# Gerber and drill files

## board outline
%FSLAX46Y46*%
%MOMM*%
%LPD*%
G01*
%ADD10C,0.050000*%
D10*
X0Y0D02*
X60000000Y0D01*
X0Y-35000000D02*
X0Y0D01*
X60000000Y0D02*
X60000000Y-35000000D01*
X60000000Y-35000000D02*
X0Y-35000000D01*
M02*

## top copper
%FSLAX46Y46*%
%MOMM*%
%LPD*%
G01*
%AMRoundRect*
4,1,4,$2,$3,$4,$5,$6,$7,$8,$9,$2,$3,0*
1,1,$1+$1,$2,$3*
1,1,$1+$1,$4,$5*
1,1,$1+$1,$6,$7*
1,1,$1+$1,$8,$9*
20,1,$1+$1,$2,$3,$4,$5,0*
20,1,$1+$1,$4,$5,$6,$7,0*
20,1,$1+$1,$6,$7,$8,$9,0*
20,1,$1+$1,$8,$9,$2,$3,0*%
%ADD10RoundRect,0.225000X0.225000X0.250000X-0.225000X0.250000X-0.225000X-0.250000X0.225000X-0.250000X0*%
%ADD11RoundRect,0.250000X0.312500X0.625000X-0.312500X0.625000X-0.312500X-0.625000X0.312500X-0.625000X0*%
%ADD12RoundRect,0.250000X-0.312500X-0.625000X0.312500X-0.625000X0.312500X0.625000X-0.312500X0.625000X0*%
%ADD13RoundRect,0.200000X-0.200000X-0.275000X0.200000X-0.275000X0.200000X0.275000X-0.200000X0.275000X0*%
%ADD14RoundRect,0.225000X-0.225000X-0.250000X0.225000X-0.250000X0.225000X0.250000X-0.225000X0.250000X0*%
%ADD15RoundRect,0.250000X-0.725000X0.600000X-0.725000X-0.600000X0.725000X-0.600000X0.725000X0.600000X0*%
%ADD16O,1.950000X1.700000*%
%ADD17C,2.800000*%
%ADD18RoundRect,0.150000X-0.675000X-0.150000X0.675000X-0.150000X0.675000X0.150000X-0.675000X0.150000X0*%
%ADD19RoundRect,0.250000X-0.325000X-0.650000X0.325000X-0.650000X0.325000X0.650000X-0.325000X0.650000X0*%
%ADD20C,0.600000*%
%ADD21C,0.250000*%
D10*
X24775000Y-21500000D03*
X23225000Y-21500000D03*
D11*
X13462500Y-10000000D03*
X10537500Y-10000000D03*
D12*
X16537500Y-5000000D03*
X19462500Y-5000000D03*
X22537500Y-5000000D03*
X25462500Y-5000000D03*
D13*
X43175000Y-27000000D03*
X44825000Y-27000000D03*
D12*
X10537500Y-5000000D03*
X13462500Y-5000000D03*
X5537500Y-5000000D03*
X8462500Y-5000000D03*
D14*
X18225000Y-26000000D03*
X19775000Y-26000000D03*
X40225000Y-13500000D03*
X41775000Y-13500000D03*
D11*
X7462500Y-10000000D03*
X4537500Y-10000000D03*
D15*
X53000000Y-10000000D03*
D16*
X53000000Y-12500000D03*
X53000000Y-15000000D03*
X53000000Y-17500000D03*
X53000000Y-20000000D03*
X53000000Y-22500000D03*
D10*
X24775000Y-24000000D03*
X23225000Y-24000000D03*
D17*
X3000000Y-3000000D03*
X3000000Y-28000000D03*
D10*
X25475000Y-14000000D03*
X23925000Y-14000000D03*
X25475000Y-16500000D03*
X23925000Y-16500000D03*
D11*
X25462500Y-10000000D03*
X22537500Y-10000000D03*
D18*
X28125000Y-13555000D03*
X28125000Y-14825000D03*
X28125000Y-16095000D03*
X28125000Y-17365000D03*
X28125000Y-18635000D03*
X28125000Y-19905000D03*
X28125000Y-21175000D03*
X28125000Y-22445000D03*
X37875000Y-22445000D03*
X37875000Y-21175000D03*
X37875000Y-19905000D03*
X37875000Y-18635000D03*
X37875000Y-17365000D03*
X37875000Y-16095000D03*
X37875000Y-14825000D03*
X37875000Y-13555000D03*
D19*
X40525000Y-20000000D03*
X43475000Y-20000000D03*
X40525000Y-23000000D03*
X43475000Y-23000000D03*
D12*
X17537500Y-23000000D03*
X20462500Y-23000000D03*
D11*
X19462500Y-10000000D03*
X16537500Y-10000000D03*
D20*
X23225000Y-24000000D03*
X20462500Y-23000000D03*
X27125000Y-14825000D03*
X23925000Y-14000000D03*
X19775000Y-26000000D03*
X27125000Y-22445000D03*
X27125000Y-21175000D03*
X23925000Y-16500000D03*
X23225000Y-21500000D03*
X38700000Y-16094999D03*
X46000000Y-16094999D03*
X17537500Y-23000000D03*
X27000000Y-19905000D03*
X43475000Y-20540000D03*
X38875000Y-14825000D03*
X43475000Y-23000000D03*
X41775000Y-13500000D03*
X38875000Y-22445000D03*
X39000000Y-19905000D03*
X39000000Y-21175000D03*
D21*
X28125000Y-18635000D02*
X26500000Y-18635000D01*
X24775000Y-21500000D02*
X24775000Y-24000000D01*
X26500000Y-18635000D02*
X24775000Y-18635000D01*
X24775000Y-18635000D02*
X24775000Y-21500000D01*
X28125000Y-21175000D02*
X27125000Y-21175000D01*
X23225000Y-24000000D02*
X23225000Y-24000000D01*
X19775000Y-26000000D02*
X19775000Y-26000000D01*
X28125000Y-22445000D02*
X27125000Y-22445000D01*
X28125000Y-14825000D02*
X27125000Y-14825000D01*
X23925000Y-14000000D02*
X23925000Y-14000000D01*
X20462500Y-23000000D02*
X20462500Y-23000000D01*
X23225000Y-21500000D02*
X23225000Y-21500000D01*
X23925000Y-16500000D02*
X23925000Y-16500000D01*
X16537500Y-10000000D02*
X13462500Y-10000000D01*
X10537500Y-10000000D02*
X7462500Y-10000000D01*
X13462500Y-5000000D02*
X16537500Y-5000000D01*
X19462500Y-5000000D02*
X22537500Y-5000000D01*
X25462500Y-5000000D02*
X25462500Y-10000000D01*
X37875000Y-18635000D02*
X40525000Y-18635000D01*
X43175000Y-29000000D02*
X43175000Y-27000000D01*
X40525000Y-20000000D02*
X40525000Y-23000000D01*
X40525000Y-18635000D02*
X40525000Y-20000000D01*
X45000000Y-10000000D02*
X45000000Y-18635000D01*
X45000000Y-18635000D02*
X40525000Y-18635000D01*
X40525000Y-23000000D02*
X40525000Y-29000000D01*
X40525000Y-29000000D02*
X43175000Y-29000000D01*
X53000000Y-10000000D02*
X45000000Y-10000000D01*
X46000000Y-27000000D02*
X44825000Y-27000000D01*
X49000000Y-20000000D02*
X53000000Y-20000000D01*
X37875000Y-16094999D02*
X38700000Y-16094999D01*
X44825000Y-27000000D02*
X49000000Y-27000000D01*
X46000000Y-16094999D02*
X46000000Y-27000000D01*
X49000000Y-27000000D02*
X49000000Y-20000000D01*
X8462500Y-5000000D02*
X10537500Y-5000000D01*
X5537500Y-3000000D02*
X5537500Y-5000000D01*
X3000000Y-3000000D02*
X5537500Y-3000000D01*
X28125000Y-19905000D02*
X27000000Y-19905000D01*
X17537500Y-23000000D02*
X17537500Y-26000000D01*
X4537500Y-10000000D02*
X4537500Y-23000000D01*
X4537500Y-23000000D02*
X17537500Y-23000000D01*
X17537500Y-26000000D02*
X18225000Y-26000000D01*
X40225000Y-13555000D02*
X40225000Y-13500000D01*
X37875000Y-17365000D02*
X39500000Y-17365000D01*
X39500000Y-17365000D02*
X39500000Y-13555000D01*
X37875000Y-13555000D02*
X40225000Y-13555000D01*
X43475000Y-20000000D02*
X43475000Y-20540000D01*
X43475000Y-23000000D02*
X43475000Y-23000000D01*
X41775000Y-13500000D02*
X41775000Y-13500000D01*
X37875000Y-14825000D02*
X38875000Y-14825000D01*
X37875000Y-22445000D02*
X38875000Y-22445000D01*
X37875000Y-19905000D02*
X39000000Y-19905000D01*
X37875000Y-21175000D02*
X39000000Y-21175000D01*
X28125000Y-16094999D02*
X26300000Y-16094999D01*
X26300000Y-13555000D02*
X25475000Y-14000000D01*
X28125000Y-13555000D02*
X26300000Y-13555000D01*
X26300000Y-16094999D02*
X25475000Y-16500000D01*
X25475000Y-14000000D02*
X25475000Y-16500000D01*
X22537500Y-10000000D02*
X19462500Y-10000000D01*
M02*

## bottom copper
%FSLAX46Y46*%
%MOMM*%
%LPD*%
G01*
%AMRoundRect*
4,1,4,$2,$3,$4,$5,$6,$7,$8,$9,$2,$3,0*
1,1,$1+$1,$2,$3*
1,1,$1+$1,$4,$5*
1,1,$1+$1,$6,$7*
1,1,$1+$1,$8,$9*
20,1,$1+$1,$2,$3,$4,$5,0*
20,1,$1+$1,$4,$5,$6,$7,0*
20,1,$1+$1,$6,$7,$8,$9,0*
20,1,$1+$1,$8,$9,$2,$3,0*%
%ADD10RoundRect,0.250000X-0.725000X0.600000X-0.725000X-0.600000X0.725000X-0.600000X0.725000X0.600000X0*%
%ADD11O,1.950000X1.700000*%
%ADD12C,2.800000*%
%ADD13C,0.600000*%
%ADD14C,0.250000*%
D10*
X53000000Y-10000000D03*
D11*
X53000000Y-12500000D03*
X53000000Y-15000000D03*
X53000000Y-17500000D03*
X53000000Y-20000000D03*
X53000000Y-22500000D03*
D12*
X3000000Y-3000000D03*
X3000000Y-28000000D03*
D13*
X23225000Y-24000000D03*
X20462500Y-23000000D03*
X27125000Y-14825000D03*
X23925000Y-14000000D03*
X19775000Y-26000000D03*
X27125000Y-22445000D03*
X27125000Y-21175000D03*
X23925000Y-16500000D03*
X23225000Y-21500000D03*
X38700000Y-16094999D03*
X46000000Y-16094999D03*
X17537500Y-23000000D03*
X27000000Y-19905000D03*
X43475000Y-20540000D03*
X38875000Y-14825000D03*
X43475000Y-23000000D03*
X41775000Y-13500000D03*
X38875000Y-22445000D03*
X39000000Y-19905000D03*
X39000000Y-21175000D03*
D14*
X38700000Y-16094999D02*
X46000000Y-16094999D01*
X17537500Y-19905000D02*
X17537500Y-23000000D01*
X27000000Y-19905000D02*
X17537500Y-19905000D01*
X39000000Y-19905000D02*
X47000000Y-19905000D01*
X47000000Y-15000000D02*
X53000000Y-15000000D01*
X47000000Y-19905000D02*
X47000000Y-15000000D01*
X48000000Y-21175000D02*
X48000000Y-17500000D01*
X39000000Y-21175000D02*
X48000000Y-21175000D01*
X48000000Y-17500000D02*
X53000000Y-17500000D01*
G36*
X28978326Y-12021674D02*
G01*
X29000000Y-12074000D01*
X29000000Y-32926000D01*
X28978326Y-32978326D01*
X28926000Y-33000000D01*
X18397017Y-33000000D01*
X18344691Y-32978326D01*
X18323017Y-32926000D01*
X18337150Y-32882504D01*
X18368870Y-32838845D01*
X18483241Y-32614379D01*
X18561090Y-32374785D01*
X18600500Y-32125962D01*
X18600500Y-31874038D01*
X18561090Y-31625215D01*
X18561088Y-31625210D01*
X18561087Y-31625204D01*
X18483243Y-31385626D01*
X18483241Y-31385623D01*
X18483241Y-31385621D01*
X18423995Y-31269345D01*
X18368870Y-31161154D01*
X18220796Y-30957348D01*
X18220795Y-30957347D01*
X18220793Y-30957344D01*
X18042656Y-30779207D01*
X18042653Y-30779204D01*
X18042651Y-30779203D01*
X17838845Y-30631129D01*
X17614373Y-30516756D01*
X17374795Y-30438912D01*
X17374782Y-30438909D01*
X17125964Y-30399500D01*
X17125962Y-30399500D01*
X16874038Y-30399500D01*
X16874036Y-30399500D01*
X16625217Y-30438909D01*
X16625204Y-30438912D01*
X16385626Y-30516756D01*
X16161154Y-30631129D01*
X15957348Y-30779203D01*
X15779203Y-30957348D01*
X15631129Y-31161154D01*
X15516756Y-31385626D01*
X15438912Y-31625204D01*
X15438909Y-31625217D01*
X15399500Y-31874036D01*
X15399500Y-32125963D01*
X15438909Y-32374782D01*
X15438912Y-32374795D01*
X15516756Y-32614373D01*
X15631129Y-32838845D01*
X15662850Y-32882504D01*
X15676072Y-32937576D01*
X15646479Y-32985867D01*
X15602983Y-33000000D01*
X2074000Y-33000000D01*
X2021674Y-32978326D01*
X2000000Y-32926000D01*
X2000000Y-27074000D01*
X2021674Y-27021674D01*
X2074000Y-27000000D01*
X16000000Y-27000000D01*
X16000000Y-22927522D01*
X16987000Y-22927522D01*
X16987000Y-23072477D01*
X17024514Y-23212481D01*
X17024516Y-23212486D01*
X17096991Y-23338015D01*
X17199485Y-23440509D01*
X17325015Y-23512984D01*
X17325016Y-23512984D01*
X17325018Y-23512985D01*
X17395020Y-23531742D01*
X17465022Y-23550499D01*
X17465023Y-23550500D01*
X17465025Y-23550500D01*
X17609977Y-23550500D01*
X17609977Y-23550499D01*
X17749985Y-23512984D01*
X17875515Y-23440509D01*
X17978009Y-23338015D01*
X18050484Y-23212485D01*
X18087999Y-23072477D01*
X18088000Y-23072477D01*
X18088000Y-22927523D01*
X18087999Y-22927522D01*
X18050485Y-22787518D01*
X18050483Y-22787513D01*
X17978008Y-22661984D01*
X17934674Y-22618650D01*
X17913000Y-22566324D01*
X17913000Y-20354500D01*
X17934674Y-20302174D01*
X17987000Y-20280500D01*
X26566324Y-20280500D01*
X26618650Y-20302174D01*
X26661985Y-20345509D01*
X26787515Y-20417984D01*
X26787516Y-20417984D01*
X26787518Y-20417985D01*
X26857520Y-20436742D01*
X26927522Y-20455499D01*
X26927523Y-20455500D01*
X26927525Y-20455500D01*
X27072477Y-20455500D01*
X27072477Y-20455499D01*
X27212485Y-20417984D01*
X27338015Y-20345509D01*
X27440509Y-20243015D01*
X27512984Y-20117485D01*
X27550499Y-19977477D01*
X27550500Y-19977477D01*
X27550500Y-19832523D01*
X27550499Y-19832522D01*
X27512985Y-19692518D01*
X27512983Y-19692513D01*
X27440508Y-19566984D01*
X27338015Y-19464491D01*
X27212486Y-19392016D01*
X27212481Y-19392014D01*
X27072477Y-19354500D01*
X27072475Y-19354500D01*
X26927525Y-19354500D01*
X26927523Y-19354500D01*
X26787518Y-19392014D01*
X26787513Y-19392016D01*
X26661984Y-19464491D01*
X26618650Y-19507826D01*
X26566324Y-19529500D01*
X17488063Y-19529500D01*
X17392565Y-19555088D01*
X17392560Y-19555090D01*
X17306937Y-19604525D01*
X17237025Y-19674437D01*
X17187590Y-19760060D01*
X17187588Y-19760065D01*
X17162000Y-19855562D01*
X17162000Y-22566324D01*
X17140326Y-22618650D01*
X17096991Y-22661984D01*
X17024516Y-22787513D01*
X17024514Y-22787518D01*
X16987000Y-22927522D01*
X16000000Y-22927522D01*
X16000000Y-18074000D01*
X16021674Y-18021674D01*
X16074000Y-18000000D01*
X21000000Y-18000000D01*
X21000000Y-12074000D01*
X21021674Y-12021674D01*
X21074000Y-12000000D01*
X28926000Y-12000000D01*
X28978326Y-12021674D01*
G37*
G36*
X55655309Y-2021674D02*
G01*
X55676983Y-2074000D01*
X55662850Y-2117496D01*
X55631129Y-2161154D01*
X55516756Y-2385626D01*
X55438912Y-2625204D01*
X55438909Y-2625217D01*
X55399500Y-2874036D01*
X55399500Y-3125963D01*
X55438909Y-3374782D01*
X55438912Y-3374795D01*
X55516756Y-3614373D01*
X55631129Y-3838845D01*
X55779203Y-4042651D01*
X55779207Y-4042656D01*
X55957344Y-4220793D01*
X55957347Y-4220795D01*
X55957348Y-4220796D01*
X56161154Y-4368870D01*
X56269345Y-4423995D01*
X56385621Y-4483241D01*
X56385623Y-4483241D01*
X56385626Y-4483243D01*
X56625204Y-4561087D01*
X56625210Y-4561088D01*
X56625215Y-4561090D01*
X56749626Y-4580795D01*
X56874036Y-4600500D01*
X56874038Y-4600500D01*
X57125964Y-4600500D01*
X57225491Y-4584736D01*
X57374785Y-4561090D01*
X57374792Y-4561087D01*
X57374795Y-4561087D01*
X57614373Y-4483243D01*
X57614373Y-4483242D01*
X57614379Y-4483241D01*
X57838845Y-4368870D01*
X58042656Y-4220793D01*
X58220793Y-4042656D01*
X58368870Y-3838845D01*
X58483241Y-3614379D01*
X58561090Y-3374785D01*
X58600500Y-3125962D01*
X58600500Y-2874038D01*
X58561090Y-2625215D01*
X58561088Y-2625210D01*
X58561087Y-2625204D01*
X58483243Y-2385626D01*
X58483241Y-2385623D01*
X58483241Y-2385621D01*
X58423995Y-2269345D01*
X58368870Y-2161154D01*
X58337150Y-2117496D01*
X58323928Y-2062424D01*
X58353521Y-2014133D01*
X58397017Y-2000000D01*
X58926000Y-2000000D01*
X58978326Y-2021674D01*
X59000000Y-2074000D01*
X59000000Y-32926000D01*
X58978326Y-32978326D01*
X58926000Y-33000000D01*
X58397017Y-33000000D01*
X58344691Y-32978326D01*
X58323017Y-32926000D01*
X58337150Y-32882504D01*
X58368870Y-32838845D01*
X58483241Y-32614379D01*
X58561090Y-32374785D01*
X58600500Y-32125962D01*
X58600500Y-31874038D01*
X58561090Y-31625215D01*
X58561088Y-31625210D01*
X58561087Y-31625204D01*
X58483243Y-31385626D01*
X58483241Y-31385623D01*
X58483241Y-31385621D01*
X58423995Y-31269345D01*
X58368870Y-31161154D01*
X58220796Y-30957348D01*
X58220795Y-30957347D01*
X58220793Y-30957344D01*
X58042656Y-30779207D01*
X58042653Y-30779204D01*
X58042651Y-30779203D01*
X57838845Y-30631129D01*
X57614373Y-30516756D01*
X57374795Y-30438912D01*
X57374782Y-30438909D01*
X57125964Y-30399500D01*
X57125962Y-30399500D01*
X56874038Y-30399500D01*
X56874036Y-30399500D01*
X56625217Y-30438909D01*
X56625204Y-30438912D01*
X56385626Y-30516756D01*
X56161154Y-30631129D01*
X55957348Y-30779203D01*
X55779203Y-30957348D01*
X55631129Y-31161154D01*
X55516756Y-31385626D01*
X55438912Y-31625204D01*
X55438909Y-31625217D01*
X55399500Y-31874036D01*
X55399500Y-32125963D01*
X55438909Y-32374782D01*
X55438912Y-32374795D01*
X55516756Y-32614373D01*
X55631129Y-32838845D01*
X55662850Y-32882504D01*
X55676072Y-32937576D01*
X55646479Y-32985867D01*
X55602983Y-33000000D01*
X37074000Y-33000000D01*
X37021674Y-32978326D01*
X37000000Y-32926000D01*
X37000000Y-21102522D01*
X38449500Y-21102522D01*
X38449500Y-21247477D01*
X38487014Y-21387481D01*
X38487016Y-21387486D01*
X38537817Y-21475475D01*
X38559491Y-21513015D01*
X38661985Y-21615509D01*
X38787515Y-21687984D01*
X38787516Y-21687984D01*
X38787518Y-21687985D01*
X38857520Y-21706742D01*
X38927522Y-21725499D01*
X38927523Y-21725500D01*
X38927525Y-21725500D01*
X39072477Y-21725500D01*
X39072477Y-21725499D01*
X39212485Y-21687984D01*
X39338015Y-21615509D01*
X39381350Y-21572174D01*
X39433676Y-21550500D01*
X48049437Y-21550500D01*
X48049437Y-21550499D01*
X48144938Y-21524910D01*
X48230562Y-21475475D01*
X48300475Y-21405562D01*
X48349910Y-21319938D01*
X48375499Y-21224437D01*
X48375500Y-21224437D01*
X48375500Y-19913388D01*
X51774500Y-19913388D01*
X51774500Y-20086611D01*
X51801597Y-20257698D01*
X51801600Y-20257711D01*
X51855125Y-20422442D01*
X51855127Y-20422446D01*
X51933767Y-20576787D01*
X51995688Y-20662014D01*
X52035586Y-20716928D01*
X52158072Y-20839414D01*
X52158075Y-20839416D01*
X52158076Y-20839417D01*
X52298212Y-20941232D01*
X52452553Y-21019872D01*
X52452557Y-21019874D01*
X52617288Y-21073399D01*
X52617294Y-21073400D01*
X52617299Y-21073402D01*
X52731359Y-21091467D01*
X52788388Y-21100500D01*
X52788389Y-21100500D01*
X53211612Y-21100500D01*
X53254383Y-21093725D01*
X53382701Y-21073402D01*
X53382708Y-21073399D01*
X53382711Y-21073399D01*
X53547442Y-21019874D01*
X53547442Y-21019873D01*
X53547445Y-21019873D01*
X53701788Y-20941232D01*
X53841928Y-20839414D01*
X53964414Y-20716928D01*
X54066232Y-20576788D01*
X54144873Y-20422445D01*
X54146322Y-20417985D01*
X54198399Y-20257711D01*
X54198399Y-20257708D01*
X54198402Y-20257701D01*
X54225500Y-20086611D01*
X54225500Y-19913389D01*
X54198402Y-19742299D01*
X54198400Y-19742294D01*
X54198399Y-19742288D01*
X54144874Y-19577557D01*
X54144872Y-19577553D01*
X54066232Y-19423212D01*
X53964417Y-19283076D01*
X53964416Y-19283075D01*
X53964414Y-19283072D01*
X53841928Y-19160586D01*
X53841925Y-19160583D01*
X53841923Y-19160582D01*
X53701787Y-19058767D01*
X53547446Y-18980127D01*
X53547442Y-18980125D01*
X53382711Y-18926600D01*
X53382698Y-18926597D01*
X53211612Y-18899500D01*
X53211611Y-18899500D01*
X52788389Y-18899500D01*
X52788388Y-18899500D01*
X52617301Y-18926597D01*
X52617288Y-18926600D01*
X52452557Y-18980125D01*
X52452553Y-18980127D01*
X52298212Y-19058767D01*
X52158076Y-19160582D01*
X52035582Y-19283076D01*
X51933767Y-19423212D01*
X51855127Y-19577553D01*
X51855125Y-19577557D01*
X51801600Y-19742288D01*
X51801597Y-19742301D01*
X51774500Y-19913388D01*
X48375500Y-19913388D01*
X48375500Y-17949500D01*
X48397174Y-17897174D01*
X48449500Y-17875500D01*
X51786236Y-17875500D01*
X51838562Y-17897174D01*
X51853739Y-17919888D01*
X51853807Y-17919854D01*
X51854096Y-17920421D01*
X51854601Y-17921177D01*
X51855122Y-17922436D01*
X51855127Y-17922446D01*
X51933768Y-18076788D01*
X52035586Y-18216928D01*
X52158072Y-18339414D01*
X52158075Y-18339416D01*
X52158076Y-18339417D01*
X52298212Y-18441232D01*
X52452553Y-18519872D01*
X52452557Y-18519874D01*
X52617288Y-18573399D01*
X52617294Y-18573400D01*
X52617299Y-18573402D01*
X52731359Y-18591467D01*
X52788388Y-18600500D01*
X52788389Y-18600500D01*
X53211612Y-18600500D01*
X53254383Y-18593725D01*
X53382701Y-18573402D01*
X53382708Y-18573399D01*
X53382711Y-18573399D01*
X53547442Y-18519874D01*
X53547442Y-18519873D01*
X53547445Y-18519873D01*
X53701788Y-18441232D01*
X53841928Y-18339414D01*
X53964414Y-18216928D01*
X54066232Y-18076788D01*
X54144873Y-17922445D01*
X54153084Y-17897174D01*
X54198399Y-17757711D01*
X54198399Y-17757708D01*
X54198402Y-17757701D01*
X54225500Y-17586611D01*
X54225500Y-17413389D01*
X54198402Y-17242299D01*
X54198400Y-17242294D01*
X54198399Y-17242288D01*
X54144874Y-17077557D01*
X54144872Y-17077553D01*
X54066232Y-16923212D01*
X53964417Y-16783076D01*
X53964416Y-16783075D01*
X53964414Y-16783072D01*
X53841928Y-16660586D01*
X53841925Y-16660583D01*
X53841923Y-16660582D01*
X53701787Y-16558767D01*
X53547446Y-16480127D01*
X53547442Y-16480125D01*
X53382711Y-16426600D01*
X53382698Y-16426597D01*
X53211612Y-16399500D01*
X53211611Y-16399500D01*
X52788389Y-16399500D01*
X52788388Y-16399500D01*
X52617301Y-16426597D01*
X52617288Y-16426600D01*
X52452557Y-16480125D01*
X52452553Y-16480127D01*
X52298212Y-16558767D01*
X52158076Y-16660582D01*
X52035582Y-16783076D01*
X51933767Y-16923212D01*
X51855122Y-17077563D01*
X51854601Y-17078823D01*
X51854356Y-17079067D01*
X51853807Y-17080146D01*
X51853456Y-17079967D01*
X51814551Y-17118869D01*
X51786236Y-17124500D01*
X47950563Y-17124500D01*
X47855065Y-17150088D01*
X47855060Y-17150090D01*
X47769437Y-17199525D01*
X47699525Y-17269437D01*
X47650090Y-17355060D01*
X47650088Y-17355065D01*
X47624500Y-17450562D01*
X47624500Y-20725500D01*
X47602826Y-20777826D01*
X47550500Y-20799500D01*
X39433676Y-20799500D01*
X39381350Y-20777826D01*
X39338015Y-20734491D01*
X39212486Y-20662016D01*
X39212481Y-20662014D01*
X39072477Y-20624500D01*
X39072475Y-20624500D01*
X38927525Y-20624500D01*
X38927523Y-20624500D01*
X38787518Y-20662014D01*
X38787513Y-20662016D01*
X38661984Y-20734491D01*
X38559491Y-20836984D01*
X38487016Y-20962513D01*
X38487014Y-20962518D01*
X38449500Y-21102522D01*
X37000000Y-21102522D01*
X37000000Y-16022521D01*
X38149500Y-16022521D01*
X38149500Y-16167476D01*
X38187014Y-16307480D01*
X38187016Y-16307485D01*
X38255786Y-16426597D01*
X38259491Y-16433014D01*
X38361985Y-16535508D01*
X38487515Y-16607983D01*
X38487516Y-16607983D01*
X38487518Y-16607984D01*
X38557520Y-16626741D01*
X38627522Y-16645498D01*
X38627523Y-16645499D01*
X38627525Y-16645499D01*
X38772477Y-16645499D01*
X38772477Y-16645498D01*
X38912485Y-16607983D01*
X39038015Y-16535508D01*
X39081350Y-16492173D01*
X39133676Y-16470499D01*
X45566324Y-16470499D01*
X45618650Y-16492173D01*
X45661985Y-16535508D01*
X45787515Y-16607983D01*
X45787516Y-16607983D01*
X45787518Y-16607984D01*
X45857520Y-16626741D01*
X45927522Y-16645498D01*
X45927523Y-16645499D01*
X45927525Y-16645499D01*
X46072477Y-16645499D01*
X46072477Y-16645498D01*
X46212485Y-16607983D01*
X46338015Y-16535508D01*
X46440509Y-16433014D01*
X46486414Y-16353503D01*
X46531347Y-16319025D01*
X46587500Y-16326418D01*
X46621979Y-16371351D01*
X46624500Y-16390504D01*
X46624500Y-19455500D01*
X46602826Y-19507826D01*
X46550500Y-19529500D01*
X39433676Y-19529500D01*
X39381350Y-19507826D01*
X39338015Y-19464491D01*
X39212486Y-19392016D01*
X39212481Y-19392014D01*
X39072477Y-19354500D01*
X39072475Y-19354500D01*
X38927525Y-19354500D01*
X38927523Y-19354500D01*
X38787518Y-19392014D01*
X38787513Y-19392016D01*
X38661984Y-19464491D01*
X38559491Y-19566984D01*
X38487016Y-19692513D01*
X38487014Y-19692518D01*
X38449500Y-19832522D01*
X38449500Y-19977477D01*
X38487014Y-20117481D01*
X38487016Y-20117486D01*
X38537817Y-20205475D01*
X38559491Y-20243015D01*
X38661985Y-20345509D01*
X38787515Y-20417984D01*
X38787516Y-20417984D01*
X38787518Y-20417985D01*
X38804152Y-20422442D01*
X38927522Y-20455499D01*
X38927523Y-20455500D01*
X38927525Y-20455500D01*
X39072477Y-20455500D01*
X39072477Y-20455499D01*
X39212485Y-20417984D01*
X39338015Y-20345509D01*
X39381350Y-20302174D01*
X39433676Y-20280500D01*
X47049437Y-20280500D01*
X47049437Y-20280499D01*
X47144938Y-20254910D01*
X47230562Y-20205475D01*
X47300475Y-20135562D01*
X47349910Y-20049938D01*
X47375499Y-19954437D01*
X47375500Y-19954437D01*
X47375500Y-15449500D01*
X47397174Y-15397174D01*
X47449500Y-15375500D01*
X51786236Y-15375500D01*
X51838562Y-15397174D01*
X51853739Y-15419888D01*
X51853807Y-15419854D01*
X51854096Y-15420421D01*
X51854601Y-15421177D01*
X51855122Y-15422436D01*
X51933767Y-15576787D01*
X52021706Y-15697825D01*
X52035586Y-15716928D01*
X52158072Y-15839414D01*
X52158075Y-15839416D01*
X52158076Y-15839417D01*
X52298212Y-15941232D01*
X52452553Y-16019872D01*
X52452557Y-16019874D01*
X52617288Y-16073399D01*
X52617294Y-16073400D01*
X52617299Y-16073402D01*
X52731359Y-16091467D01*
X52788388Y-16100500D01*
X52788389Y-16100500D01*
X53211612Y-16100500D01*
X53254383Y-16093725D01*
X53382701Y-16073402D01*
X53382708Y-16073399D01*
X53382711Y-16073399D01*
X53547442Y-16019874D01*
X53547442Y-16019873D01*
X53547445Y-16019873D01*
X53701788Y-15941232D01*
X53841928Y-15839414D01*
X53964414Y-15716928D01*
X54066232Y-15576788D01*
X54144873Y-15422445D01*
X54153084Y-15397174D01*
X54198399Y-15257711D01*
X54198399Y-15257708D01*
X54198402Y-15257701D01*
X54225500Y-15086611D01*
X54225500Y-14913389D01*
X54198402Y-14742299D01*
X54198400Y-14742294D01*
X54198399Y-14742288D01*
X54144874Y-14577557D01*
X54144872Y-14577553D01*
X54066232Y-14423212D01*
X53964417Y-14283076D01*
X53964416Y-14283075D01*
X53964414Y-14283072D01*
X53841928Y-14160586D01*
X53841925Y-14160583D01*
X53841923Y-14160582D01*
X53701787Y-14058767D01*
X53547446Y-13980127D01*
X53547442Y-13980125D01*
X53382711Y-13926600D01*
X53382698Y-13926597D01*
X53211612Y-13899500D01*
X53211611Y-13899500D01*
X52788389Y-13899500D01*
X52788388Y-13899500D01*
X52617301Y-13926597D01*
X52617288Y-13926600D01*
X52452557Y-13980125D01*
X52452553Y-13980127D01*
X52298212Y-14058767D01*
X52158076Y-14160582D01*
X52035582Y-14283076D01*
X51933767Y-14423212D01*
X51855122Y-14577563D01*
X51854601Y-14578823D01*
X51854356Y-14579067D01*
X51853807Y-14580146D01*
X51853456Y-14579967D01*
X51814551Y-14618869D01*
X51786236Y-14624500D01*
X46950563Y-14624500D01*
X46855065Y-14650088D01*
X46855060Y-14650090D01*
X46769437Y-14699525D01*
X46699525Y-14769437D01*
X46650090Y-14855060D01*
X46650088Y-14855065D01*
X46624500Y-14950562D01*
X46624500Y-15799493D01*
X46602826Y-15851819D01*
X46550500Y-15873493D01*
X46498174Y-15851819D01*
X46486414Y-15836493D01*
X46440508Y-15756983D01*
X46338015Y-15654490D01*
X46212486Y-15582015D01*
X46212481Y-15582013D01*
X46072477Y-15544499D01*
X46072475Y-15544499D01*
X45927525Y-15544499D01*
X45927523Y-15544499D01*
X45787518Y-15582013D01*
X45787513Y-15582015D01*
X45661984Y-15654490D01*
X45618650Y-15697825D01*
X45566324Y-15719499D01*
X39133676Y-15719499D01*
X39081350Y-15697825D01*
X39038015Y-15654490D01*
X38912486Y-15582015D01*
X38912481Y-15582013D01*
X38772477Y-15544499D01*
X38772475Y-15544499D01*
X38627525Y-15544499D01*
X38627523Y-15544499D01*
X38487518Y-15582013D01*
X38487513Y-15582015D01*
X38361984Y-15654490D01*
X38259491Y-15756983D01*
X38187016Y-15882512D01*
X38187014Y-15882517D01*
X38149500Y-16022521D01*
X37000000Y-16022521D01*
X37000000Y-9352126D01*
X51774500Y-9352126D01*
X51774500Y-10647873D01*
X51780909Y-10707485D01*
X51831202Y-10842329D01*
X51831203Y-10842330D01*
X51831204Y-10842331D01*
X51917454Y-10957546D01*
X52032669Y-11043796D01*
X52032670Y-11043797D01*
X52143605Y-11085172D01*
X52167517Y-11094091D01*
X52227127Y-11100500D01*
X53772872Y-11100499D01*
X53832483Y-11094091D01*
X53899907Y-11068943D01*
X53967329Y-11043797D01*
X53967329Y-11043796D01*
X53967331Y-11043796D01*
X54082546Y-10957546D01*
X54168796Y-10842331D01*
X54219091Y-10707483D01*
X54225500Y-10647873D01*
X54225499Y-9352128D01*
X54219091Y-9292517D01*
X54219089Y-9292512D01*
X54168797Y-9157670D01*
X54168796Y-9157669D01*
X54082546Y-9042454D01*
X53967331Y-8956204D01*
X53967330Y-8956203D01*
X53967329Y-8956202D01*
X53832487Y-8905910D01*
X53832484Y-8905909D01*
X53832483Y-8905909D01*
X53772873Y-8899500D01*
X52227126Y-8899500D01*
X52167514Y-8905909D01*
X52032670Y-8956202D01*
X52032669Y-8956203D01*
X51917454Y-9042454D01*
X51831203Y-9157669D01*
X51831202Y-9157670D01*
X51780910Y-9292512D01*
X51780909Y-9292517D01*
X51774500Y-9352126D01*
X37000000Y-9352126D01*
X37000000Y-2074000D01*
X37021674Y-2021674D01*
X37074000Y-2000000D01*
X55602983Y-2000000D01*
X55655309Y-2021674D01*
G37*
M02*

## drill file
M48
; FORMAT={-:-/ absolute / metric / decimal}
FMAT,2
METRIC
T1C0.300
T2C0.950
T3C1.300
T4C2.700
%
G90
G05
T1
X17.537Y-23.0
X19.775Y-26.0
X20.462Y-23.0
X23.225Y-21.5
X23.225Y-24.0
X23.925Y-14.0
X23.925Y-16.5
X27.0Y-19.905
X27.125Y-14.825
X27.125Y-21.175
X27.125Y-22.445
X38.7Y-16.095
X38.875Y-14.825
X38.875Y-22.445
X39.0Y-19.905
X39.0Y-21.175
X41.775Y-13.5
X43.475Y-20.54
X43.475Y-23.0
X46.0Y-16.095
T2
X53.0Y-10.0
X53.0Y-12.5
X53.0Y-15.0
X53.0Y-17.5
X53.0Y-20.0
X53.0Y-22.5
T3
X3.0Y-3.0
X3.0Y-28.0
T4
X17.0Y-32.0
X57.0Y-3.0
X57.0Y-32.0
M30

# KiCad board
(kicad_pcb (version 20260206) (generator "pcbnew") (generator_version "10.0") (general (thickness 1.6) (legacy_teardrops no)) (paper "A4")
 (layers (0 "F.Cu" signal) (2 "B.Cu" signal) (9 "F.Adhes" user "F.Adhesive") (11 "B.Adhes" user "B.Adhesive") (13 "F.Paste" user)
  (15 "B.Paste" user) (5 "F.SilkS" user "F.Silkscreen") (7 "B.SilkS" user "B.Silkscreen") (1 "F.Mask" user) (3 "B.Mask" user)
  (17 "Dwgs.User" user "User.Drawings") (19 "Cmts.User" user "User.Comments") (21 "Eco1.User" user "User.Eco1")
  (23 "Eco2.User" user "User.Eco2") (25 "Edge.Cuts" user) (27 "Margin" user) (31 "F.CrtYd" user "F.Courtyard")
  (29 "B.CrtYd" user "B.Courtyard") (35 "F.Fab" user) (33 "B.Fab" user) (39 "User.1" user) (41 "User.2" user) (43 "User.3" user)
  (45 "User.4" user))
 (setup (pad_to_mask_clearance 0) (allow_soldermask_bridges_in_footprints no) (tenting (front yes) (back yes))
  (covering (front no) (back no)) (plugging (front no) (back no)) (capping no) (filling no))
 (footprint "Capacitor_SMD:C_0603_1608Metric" (layer "F.Cu") (at 24 21.5 180)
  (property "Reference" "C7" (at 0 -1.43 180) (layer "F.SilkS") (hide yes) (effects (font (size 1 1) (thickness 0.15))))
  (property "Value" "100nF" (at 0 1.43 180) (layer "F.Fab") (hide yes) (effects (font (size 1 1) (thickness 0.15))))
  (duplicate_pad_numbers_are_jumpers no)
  (pad "1" smd roundrect (at -0.775 0 180) (size 0.9 0.95) (layers "F.Cu" "F.Mask" "F.Paste") (roundrect_rratio 0.25) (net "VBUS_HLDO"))
  (pad "2" smd roundrect (at 0.775 0 180) (size 0.9 0.95) (layers "F.Cu" "F.Mask" "F.Paste") (roundrect_rratio 0.25) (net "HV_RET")))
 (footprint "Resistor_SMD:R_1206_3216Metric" (layer "F.Cu") (at 12 10 180)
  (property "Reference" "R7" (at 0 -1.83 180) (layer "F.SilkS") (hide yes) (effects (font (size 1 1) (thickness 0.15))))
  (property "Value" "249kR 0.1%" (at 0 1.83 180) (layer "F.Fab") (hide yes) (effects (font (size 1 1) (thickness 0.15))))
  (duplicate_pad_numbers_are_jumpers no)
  (pad "1" smd roundrect (at -1.4625 0 180) (size 1.125 1.75) (layers "F.Cu" "F.Mask" "F.Paste") (roundrect_rratio 0.222222)
   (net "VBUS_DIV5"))
  (pad "2" smd roundrect (at 1.4625 0 180) (size 1.125 1.75) (layers "F.Cu" "F.Mask" "F.Paste") (roundrect_rratio 0.222222)
   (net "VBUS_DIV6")))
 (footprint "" (layer "F.Cu") (at 57 32)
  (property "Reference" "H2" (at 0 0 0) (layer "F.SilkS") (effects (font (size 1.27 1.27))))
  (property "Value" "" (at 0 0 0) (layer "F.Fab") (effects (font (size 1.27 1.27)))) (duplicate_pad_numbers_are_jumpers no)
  (pad "" np_thru_hole circle (at 0 0) (size 2.7 2.7) (drill 2.7) (layers "*.Cu")))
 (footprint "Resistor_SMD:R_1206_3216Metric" (layer "F.Cu") (at 18 5)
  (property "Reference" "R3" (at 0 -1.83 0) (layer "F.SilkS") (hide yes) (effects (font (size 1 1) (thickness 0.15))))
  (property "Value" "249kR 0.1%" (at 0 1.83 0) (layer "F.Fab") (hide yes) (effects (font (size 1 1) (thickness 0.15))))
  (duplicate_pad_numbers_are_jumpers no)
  (pad "1" smd roundrect (at -1.4625 0) (size 1.125 1.75) (layers "F.Cu" "F.Mask" "F.Paste") (roundrect_rratio 0.222222) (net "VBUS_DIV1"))
  (pad "2" smd roundrect (at 1.4625 0) (size 1.125 1.75) (layers "F.Cu" "F.Mask" "F.Paste") (roundrect_rratio 0.222222) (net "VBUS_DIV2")))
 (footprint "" (layer "F.Cu") (at 57 3)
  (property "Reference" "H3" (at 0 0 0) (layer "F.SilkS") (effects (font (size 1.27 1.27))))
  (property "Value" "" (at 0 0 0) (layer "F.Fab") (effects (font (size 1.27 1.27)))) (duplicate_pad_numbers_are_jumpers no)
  (pad "" np_thru_hole circle (at 0 0) (size 2.7 2.7) (drill 2.7) (layers "*.Cu")))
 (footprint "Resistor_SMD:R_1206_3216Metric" (layer "F.Cu") (at 24 5)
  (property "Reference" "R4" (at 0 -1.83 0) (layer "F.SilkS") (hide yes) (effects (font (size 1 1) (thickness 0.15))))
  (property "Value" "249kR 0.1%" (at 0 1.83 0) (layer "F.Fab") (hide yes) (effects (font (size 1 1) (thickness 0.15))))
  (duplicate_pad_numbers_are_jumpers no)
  (pad "1" smd roundrect (at -1.4625 0) (size 1.125 1.75) (layers "F.Cu" "F.Mask" "F.Paste") (roundrect_rratio 0.222222) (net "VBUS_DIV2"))
  (pad "2" smd roundrect (at 1.4625 0) (size 1.125 1.75) (layers "F.Cu" "F.Mask" "F.Paste") (roundrect_rratio 0.222222) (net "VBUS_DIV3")))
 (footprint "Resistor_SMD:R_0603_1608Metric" (layer "F.Cu") (at 44 27)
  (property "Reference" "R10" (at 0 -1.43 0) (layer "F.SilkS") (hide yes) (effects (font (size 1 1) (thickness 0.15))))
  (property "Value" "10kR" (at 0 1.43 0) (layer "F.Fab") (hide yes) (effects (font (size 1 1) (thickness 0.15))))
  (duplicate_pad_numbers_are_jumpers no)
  (pad "1" smd roundrect (at -0.825 0) (size 0.8 0.95) (layers "F.Cu" "F.Mask" "F.Paste") (roundrect_rratio 0.25) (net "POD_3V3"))
  (pad "2" smd roundrect (at 0.825 0) (size 0.8 0.95) (layers "F.Cu" "F.Mask" "F.Paste") (roundrect_rratio 0.25) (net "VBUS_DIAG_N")))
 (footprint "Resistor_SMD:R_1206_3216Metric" (layer "F.Cu") (at 12 5)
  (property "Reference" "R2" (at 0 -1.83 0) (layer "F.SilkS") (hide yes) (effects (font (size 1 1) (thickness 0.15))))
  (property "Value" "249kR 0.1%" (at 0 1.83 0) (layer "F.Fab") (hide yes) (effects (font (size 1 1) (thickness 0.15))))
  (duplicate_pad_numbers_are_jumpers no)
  (pad "1" smd roundrect (at -1.4625 0) (size 1.125 1.75) (layers "F.Cu" "F.Mask" "F.Paste") (roundrect_rratio 0.222222) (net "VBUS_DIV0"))
  (pad "2" smd roundrect (at 1.4625 0) (size 1.125 1.75) (layers "F.Cu" "F.Mask" "F.Paste") (roundrect_rratio 0.222222) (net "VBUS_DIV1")))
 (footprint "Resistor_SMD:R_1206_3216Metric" (layer "F.Cu") (at 7 5)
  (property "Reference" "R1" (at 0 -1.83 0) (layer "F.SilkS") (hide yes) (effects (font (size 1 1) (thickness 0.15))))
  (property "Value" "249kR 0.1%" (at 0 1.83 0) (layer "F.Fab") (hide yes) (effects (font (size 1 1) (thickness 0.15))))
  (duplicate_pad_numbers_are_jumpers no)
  (pad "1" smd roundrect (at -1.4625 0) (size 1.125 1.75) (layers "F.Cu" "F.Mask" "F.Paste") (roundrect_rratio 0.222222) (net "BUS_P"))
  (pad "2" smd roundrect (at 1.4625 0) (size 1.125 1.75) (layers "F.Cu" "F.Mask" "F.Paste") (roundrect_rratio 0.222222) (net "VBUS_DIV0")))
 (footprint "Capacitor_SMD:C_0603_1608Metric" (layer "F.Cu") (at 19 26)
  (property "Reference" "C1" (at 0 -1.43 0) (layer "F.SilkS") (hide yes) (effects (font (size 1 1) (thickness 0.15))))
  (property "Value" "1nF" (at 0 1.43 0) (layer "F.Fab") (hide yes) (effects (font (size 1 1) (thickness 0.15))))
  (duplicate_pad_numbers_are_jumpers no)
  (pad "1" smd roundrect (at -0.775 0) (size 0.9 0.95) (layers "F.Cu" "F.Mask" "F.Paste") (roundrect_rratio 0.25) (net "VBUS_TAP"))
  (pad "2" smd roundrect (at 0.775 0) (size 0.9 0.95) (layers "F.Cu" "F.Mask" "F.Paste") (roundrect_rratio 0.25) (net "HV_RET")))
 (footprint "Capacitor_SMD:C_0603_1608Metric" (layer "F.Cu") (at 41 13.5)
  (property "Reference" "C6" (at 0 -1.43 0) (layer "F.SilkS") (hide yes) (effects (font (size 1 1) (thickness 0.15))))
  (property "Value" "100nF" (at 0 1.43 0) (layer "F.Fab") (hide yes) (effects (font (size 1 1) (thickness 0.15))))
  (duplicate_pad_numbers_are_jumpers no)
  (pad "1" smd roundrect (at -0.775 0) (size 0.9 0.95) (layers "F.Cu" "F.Mask" "F.Paste") (roundrect_rratio 0.25) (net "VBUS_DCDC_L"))
  (pad "2" smd roundrect (at 0.775 0) (size 0.9 0.95) (layers "F.Cu" "F.Mask" "F.Paste") (roundrect_rratio 0.25) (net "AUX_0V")))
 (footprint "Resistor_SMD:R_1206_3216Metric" (layer "F.Cu") (at 6 10 180)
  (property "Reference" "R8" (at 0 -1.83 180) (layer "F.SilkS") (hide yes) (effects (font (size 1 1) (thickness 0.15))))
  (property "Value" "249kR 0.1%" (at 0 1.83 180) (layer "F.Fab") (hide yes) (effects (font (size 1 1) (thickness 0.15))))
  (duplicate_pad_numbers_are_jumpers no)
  (pad "1" smd roundrect (at -1.4625 0 180) (size 1.125 1.75) (layers "F.Cu" "F.Mask" "F.Paste") (roundrect_rratio 0.222222)
   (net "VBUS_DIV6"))
  (pad "2" smd roundrect (at 1.4625 0 180) (size 1.125 1.75) (layers "F.Cu" "F.Mask" "F.Paste") (roundrect_rratio 0.222222) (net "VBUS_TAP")))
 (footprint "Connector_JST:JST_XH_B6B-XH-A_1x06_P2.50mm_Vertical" (layer "F.Cu") (at 53 10 -90)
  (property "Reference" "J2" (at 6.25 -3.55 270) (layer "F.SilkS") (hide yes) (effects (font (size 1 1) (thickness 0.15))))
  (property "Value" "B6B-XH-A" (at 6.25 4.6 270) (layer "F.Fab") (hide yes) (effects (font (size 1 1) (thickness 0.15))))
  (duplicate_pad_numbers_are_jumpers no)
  (pad "1" thru_hole roundrect (at 0 0 270) (size 1.7 1.95) (drill 0.95) (layers "*.Cu" "*.Mask") (remove_unused_layers no)
   (roundrect_rratio 0.147059) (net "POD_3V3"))
  (pad "2" thru_hole oval (at 2.5 0 270) (size 1.7 1.95) (drill 0.95) (layers "*.Cu" "*.Mask") (remove_unused_layers no) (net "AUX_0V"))
  (pad "3" thru_hole oval (at 5 0 270) (size 1.7 1.95) (drill 0.95) (layers "*.Cu" "*.Mask") (remove_unused_layers no) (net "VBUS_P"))
  (pad "4" thru_hole oval (at 7.5 0 270) (size 1.7 1.95) (drill 0.95) (layers "*.Cu" "*.Mask") (remove_unused_layers no) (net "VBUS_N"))
  (pad "5" thru_hole oval (at 10 0 270) (size 1.7 1.95) (drill 0.95) (layers "*.Cu" "*.Mask") (remove_unused_layers no) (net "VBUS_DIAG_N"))
  (pad "6" thru_hole oval (at 12.5 0 270) (size 1.7 1.95) (drill 0.95) (layers "*.Cu" "*.Mask") (remove_unused_layers no) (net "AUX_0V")))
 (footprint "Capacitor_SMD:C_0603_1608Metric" (layer "F.Cu") (at 24 24 180)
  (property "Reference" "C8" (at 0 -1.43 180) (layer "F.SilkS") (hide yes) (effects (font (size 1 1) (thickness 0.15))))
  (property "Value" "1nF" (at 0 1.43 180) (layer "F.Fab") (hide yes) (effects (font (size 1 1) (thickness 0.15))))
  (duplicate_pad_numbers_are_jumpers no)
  (pad "1" smd roundrect (at -0.775 0 180) (size 0.9 0.95) (layers "F.Cu" "F.Mask" "F.Paste") (roundrect_rratio 0.25) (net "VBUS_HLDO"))
  (pad "2" smd roundrect (at 0.775 0 180) (size 0.9 0.95) (layers "F.Cu" "F.Mask" "F.Paste") (roundrect_rratio 0.25) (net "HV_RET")))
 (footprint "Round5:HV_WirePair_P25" (layer "F.Cu") (at 3 3)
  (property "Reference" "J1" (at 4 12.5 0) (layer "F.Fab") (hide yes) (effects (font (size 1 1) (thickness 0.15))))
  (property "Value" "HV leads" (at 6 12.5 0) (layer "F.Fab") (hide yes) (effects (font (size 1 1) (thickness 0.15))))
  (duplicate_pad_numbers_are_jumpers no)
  (pad "1" thru_hole circle (at 0 0) (size 2.8 2.8) (drill 1.3) (layers "*.Cu" "*.Mask") (remove_unused_layers no) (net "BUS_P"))
  (pad "2" thru_hole circle (at 0 25) (size 2.8 2.8) (drill 1.3) (layers "*.Cu" "*.Mask") (remove_unused_layers no) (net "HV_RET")))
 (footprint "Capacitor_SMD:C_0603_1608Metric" (layer "F.Cu") (at 24.7 14 180)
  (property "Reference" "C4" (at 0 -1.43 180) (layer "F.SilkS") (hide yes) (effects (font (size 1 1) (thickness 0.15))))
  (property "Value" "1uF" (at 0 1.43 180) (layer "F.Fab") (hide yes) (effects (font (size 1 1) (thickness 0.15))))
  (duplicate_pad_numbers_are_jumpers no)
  (pad "1" smd roundrect (at -0.775 0 180) (size 0.9 0.95) (layers "F.Cu" "F.Mask" "F.Paste") (roundrect_rratio 0.25) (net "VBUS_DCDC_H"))
  (pad "2" smd roundrect (at 0.775 0 180) (size 0.9 0.95) (layers "F.Cu" "F.Mask" "F.Paste") (roundrect_rratio 0.25) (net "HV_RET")))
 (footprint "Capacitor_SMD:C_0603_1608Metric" (layer "F.Cu") (at 24.7 16.5 180)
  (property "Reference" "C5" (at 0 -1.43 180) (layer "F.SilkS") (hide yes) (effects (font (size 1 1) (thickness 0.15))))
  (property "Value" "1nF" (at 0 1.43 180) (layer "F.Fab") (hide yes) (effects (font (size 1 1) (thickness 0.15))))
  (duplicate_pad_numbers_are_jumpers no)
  (pad "1" smd roundrect (at -0.775 0 180) (size 0.9 0.95) (layers "F.Cu" "F.Mask" "F.Paste") (roundrect_rratio 0.25) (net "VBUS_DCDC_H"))
  (pad "2" smd roundrect (at 0.775 0 180) (size 0.9 0.95) (layers "F.Cu" "F.Mask" "F.Paste") (roundrect_rratio 0.25) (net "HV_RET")))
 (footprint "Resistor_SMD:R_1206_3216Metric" (layer "F.Cu") (at 24 10 180)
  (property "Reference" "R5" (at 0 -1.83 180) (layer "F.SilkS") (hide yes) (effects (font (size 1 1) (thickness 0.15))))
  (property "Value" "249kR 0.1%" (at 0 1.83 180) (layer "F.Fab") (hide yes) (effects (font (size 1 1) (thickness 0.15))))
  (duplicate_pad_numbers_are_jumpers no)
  (pad "1" smd roundrect (at -1.4625 0 180) (size 1.125 1.75) (layers "F.Cu" "F.Mask" "F.Paste") (roundrect_rratio 0.222222)
   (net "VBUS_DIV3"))
  (pad "2" smd roundrect (at 1.4625 0 180) (size 1.125 1.75) (layers "F.Cu" "F.Mask" "F.Paste") (roundrect_rratio 0.222222)
   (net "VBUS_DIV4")))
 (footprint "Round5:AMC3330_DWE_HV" (layer "F.Cu") (at 33 18)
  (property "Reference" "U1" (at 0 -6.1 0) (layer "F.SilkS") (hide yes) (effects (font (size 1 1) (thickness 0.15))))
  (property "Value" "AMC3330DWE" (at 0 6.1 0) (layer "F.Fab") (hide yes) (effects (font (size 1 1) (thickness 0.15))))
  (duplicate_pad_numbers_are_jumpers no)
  (pad "1" smd roundrect (at -4.875 -4.445) (size 1.65 0.6) (layers "F.Cu" "F.Mask" "F.Paste") (roundrect_rratio 0.25) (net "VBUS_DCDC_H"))
  (pad "2" smd roundrect (at -4.875 -3.175) (size 1.65 0.6) (layers "F.Cu" "F.Mask" "F.Paste") (roundrect_rratio 0.25) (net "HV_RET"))
  (pad "3" smd roundrect (at -4.875 -1.905) (size 1.65 0.6) (layers "F.Cu" "F.Mask" "F.Paste") (roundrect_rratio 0.25) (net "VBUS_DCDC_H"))
  (pad "4" smd roundrect (at -4.875 -0.635) (size 1.65 0.6) (layers "F.Cu" "F.Mask" "F.Paste") (roundrect_rratio 0.25)
   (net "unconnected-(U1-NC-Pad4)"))
  (pad "5" smd roundrect (at -4.875 0.635) (size 1.65 0.6) (layers "F.Cu" "F.Mask" "F.Paste") (roundrect_rratio 0.25) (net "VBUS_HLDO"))
  (pad "6" smd roundrect (at -4.875 1.905) (size 1.65 0.6) (layers "F.Cu" "F.Mask" "F.Paste") (roundrect_rratio 0.25) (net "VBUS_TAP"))
  (pad "7" smd roundrect (at -4.875 3.175) (size 1.65 0.6) (layers "F.Cu" "F.Mask" "F.Paste") (roundrect_rratio 0.25) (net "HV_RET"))
  (pad "8" smd roundrect (at -4.875 4.445) (size 1.65 0.6) (layers "F.Cu" "F.Mask" "F.Paste") (roundrect_rratio 0.25) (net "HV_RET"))
  (pad "9" smd roundrect (at 4.875 4.445) (size 1.65 0.6) (layers "F.Cu" "F.Mask" "F.Paste") (roundrect_rratio 0.25) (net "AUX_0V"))
  (pad "10" smd roundrect (at 4.875 3.175) (size 1.65 0.6) (layers "F.Cu" "F.Mask" "F.Paste") (roundrect_rratio 0.25) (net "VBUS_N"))
  (pad "11" smd roundrect (at 4.875 1.905) (size 1.65 0.6) (layers "F.Cu" "F.Mask" "F.Paste") (roundrect_rratio 0.25) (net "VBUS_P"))
  (pad "12" smd roundrect (at 4.875 0.635) (size 1.65 0.6) (layers "F.Cu" "F.Mask" "F.Paste") (roundrect_rratio 0.25) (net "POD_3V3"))
  (pad "13" smd roundrect (at 4.875 -0.635) (size 1.65 0.6) (layers "F.Cu" "F.Mask" "F.Paste") (roundrect_rratio 0.25) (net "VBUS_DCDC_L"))
  (pad "14" smd roundrect (at 4.875 -1.905) (size 1.65 0.6) (layers "F.Cu" "F.Mask" "F.Paste") (roundrect_rratio 0.25) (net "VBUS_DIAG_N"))
  (pad "15" smd roundrect (at 4.875 -3.175) (size 1.65 0.6) (layers "F.Cu" "F.Mask" "F.Paste") (roundrect_rratio 0.25) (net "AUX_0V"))
  (pad "16" smd roundrect (at 4.875 -4.445) (size 1.65 0.6) (layers "F.Cu" "F.Mask" "F.Paste") (roundrect_rratio 0.25) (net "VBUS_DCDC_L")))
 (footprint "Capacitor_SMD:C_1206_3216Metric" (layer "F.Cu") (at 42 20)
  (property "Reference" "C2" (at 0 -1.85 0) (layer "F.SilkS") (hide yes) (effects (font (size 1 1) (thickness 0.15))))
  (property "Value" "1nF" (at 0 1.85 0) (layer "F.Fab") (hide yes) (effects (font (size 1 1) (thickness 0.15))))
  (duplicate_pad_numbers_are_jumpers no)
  (pad "1" smd roundrect (at -1.475 0) (size 1.15 1.8) (layers "F.Cu" "F.Mask" "F.Paste") (roundrect_rratio 0.217391) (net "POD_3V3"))
  (pad "2" smd roundrect (at 1.475 0) (size 1.15 1.8) (layers "F.Cu" "F.Mask" "F.Paste") (roundrect_rratio 0.217391) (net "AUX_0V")))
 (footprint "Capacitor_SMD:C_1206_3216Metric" (layer "F.Cu") (at 42 23)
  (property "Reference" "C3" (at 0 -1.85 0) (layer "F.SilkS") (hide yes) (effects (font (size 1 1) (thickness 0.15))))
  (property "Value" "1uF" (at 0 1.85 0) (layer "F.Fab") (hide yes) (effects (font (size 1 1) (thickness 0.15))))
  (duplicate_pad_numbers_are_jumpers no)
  (pad "1" smd roundrect (at -1.475 0) (size 1.15 1.8) (layers "F.Cu" "F.Mask" "F.Paste") (roundrect_rratio 0.217391) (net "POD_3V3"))
  (pad "2" smd roundrect (at 1.475 0) (size 1.15 1.8) (layers "F.Cu" "F.Mask" "F.Paste") (roundrect_rratio 0.217391) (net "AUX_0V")))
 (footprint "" (layer "F.Cu") (at 17 32)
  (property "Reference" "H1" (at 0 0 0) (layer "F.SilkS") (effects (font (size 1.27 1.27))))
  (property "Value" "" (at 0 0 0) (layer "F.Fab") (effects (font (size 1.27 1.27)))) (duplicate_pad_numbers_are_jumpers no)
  (pad "" np_thru_hole circle (at 0 0) (size 2.7 2.7) (drill 2.7) (layers "*.Cu")))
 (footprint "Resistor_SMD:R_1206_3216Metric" (layer "F.Cu") (at 19 23)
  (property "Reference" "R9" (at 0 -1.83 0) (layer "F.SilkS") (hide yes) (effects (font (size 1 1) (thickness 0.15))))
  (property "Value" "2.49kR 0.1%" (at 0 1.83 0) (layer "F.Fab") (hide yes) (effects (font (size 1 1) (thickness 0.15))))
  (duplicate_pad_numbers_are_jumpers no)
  (pad "1" smd roundrect (at -1.4625 0) (size 1.125 1.75) (layers "F.Cu" "F.Mask" "F.Paste") (roundrect_rratio 0.222222) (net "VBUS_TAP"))
  (pad "2" smd roundrect (at 1.4625 0) (size 1.125 1.75) (layers "F.Cu" "F.Mask" "F.Paste") (roundrect_rratio 0.222222) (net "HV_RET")))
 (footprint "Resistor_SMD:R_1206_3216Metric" (layer "F.Cu") (at 18 10 180)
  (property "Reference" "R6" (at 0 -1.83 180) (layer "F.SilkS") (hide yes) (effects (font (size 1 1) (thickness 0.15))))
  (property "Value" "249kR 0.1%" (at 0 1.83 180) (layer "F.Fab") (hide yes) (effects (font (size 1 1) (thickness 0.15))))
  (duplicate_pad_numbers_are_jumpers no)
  (pad "1" smd roundrect (at -1.4625 0 180) (size 1.125 1.75) (layers "F.Cu" "F.Mask" "F.Paste") (roundrect_rratio 0.222222)
   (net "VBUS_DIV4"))
  (pad "2" smd roundrect (at 1.4625 0 180) (size 1.125 1.75) (layers "F.Cu" "F.Mask" "F.Paste") (roundrect_rratio 0.222222)
   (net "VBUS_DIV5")))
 (gr_line (start 0 0) (end 60 0) (stroke (width 0.05) (type default)) (layer "Edge.Cuts"))
 (gr_line (start 0 35) (end 0 0) (stroke (width 0.05) (type default)) (layer "Edge.Cuts"))
 (gr_line (start 60 0) (end 60 35) (stroke (width 0.05) (type default)) (layer "Edge.Cuts"))
 (gr_line (start 60 35) (end 0 35) (stroke (width 0.05) (type default)) (layer "Edge.Cuts"))
 (segment (start 28.125 18.635) (end 26.5 18.635) (width 0.25) (layer "F.Cu") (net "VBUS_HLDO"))
 (segment (start 24.775 21.5) (end 24.775 24) (width 0.25) (layer "F.Cu") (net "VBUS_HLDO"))
 (segment (start 26.5 18.635) (end 24.775 18.635) (width 0.25) (layer "F.Cu") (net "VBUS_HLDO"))
 (segment (start 24.775 18.635) (end 24.775 21.5) (width 0.25) (layer "F.Cu") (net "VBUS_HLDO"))
 (segment (start 28.125 21.175) (end 27.125 21.175) (width 0.25) (layer "F.Cu") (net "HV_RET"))
 (segment (start 23.225 24) (end 23.225 24) (width 0.25) (layer "F.Cu") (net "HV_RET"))
 (segment (start 19.775 26) (end 19.775 26) (width 0.25) (layer "F.Cu") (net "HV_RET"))
 (segment (start 28.125 22.445) (end 27.125 22.445) (width 0.25) (layer "F.Cu") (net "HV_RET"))
 (segment (start 28.125 14.825) (end 27.125 14.825) (width 0.25) (layer "F.Cu") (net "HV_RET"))
 (segment (start 23.925 14) (end 23.925 14) (width 0.25) (layer "F.Cu") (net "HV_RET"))
 (segment (start 20.4625 23) (end 20.4625 23) (width 0.25) (layer "F.Cu") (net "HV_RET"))
 (segment (start 23.225 21.5) (end 23.225 21.5) (width 0.25) (layer "F.Cu") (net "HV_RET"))
 (segment (start 23.925 16.5) (end 23.925 16.5) (width 0.25) (layer "F.Cu") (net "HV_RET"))
 (via (at 23.225 24) (size 0.6) (drill 0.3) (layers "F.Cu" "B.Cu") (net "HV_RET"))
 (via (at 20.4625 23) (size 0.6) (drill 0.3) (layers "F.Cu" "B.Cu") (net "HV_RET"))
 (via (at 27.125 14.825) (size 0.6) (drill 0.3) (layers "F.Cu" "B.Cu") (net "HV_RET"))
 (via (at 23.925 14) (size 0.6) (drill 0.3) (layers "F.Cu" "B.Cu") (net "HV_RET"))
 (via (at 19.775 26) (size 0.6) (drill 0.3) (layers "F.Cu" "B.Cu") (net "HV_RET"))
 (via (at 27.125 22.445) (size 0.6) (drill 0.3) (layers "F.Cu" "B.Cu") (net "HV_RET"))
 (via (at 27.125 21.175) (size 0.6) (drill 0.3) (layers "F.Cu" "B.Cu") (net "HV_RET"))
 (via (at 23.925 16.5) (size 0.6) (drill 0.3) (layers "F.Cu" "B.Cu") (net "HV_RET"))
 (via (at 23.225 21.5) (size 0.6) (drill 0.3) (layers "F.Cu" "B.Cu") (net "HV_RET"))
 (segment (start 16.5375 10) (end 13.4625 10) (width 0.25) (layer "F.Cu") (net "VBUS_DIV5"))
 (segment (start 10.5375 10) (end 7.4625 10) (width 0.25) (layer "F.Cu") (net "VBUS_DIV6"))
 (segment (start 13.4625 5) (end 16.5375 5) (width 0.25) (layer "F.Cu") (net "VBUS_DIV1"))
 (segment (start 19.4625 5) (end 22.5375 5) (width 0.25) (layer "F.Cu") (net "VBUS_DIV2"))
 (segment (start 25.4625 5) (end 25.4625 10) (width 0.25) (layer "F.Cu") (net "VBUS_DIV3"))
 (segment (start 37.875 18.635) (end 40.525 18.635) (width 0.25) (layer "F.Cu") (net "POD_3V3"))
 (segment (start 43.175 29) (end 43.175 27) (width 0.25) (layer "F.Cu") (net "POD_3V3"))
 (segment (start 40.525 20) (end 40.525 23) (width 0.25) (layer "F.Cu") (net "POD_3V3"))
 (segment (start 40.525 18.635) (end 40.525 20) (width 0.25) (layer "F.Cu") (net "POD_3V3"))
 (segment (start 45 10) (end 45 18.635) (width 0.25) (layer "F.Cu") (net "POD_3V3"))
 (segment (start 45 18.635) (end 40.525 18.635) (width 0.25) (layer "F.Cu") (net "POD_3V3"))
 (segment (start 40.525 23) (end 40.525 29) (width 0.25) (layer "F.Cu") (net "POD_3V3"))
 (segment (start 40.525 29) (end 43.175 29) (width 0.25) (layer "F.Cu") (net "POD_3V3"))
 (segment (start 53 10) (end 45 10) (width 0.25) (layer "F.Cu") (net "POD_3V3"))
 (segment (start 46 27) (end 44.825 27) (width 0.25) (layer "F.Cu") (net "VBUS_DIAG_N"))
 (segment (start 49 20) (end 53 20) (width 0.25) (layer "F.Cu") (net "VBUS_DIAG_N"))
 (segment (start 37.875 16.094999) (end 38.7 16.094999) (width 0.25) (layer "F.Cu") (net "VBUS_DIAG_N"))
 (segment (start 44.825 27) (end 49 27) (width 0.25) (layer "F.Cu") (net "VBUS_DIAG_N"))
 (segment (start 46 16.094999) (end 46 27) (width 0.25) (layer "F.Cu") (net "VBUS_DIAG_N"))
 (segment (start 49 27) (end 49 20) (width 0.25) (layer "F.Cu") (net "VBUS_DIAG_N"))
 (via (at 38.7 16.094999) (size 0.6) (drill 0.3) (layers "F.Cu" "B.Cu") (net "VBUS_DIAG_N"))
 (via (at 46 16.094999) (size 0.6) (drill 0.3) (layers "F.Cu" "B.Cu") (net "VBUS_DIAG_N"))
 (segment (start 38.7 16.094999) (end 46 16.094999) (width 0.25) (layer "B.Cu") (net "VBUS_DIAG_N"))
 (segment (start 8.4625 5) (end 10.5375 5) (width 0.25) (layer "F.Cu") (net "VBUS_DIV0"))
 (segment (start 5.5375 3) (end 5.5375 5) (width 0.25) (layer "F.Cu") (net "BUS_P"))
 (segment (start 3 3) (end 5.5375 3) (width 0.25) (layer "F.Cu") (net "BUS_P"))
 (segment (start 28.125 19.905) (end 27 19.905) (width 0.25) (layer "F.Cu") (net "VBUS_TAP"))
 (segment (start 17.5375 23) (end 17.5375 26) (width 0.25) (layer "F.Cu") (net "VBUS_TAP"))
 (segment (start 4.5375 10) (end 4.5375 23) (width 0.25) (layer "F.Cu") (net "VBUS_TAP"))
 (segment (start 4.5375 23) (end 17.5375 23) (width 0.25) (layer "F.Cu") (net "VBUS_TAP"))
 (segment (start 17.5375 26) (end 18.225 26) (width 0.25) (layer "F.Cu") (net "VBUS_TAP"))
 (via (at 17.5375 23) (size 0.6) (drill 0.3) (layers "F.Cu" "B.Cu") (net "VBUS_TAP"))
 (via (at 27 19.905) (size 0.6) (drill 0.3) (layers "F.Cu" "B.Cu") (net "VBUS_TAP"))
 (segment (start 17.5375 19.905) (end 17.5375 23) (width 0.25) (layer "B.Cu") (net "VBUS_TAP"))
 (segment (start 27 19.905) (end 17.5375 19.905) (width 0.25) (layer "B.Cu") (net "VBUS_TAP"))
 (segment (start 40.225 13.555) (end 40.225 13.5) (width 0.25) (layer "F.Cu") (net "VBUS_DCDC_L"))
 (segment (start 37.875 17.365) (end 39.5 17.365) (width 0.25) (layer "F.Cu") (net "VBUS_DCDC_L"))
 (segment (start 39.5 17.365) (end 39.5 13.555) (width 0.25) (layer "F.Cu") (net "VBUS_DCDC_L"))
 (segment (start 37.875 13.555) (end 40.225 13.555) (width 0.25) (layer "F.Cu") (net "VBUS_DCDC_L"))
 (segment (start 43.475 20) (end 43.475 20.54) (width 0.25) (layer "F.Cu") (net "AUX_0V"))
 (segment (start 43.475 23) (end 43.475 23) (width 0.25) (layer "F.Cu") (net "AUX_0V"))
 (segment (start 41.775 13.5) (end 41.775 13.5) (width 0.25) (layer "F.Cu") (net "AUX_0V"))
 (segment (start 37.875 14.825) (end 38.875 14.825) (width 0.25) (layer "F.Cu") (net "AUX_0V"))
 (segment (start 37.875 22.445) (end 38.875 22.445) (width 0.25) (layer "F.Cu") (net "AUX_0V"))
 (via (at 43.475 20.54) (size 0.6) (drill 0.3) (layers "F.Cu" "B.Cu") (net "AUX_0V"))
 (via (at 38.875 14.825) (size 0.6) (drill 0.3) (layers "F.Cu" "B.Cu") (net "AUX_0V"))
 (via (at 43.475 23) (size 0.6) (drill 0.3) (layers "F.Cu" "B.Cu") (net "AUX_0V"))
 (via (at 41.775 13.5) (size 0.6) (drill 0.3) (layers "F.Cu" "B.Cu") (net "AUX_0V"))
 (via (at 38.875 22.445) (size 0.6) (drill 0.3) (layers "F.Cu" "B.Cu") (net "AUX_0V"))
 (segment (start 37.875 19.905) (end 39 19.905) (width 0.25) (layer "F.Cu") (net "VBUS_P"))
 (via (at 39 19.905) (size 0.6) (drill 0.3) (layers "F.Cu" "B.Cu") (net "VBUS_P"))
 (segment (start 39 19.905) (end 47 19.905) (width 0.25) (layer "B.Cu") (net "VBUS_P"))
 (segment (start 47 15) (end 53 15) (width 0.25) (layer "B.Cu") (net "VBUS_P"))
 (segment (start 47 19.905) (end 47 15) (width 0.25) (layer "B.Cu") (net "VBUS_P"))
 (segment (start 37.875 21.175) (end 39 21.175) (width 0.25) (layer "F.Cu") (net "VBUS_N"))
 (via (at 39 21.175) (size 0.6) (drill 0.3) (layers "F.Cu" "B.Cu") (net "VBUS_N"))
 (segment (start 48 21.175) (end 48 17.5) (width 0.25) (layer "B.Cu") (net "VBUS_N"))
 (segment (start 39 21.175) (end 48 21.175) (width 0.25) (layer "B.Cu") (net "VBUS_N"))
 (segment (start 48 17.5) (end 53 17.5) (width 0.25) (layer "B.Cu") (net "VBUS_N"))
 (segment (start 28.125 16.094999) (end 26.3 16.094999) (width 0.25) (layer "F.Cu") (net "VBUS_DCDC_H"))
 (segment (start 26.3 13.555) (end 25.475 14) (width 0.25) (layer "F.Cu") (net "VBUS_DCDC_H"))
 (segment (start 28.125 13.555) (end 26.3 13.555) (width 0.25) (layer "F.Cu") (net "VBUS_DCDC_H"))
 (segment (start 26.3 16.094999) (end 25.475 16.5) (width 0.25) (layer "F.Cu") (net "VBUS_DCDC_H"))
 (segment (start 25.475 14) (end 25.475 16.5) (width 0.25) (layer "F.Cu") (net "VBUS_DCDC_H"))
 (segment (start 22.5375 10) (end 19.4625 10) (width 0.25) (layer "F.Cu") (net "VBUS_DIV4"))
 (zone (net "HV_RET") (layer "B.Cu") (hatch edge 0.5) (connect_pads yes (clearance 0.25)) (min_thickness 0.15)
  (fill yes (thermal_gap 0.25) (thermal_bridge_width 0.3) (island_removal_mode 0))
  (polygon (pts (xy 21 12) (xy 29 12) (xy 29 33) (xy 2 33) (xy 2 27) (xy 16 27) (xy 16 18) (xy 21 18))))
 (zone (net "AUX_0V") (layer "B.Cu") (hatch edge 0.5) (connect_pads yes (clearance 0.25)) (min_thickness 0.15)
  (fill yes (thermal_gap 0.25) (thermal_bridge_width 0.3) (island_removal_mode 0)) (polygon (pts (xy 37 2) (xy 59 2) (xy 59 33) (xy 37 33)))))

